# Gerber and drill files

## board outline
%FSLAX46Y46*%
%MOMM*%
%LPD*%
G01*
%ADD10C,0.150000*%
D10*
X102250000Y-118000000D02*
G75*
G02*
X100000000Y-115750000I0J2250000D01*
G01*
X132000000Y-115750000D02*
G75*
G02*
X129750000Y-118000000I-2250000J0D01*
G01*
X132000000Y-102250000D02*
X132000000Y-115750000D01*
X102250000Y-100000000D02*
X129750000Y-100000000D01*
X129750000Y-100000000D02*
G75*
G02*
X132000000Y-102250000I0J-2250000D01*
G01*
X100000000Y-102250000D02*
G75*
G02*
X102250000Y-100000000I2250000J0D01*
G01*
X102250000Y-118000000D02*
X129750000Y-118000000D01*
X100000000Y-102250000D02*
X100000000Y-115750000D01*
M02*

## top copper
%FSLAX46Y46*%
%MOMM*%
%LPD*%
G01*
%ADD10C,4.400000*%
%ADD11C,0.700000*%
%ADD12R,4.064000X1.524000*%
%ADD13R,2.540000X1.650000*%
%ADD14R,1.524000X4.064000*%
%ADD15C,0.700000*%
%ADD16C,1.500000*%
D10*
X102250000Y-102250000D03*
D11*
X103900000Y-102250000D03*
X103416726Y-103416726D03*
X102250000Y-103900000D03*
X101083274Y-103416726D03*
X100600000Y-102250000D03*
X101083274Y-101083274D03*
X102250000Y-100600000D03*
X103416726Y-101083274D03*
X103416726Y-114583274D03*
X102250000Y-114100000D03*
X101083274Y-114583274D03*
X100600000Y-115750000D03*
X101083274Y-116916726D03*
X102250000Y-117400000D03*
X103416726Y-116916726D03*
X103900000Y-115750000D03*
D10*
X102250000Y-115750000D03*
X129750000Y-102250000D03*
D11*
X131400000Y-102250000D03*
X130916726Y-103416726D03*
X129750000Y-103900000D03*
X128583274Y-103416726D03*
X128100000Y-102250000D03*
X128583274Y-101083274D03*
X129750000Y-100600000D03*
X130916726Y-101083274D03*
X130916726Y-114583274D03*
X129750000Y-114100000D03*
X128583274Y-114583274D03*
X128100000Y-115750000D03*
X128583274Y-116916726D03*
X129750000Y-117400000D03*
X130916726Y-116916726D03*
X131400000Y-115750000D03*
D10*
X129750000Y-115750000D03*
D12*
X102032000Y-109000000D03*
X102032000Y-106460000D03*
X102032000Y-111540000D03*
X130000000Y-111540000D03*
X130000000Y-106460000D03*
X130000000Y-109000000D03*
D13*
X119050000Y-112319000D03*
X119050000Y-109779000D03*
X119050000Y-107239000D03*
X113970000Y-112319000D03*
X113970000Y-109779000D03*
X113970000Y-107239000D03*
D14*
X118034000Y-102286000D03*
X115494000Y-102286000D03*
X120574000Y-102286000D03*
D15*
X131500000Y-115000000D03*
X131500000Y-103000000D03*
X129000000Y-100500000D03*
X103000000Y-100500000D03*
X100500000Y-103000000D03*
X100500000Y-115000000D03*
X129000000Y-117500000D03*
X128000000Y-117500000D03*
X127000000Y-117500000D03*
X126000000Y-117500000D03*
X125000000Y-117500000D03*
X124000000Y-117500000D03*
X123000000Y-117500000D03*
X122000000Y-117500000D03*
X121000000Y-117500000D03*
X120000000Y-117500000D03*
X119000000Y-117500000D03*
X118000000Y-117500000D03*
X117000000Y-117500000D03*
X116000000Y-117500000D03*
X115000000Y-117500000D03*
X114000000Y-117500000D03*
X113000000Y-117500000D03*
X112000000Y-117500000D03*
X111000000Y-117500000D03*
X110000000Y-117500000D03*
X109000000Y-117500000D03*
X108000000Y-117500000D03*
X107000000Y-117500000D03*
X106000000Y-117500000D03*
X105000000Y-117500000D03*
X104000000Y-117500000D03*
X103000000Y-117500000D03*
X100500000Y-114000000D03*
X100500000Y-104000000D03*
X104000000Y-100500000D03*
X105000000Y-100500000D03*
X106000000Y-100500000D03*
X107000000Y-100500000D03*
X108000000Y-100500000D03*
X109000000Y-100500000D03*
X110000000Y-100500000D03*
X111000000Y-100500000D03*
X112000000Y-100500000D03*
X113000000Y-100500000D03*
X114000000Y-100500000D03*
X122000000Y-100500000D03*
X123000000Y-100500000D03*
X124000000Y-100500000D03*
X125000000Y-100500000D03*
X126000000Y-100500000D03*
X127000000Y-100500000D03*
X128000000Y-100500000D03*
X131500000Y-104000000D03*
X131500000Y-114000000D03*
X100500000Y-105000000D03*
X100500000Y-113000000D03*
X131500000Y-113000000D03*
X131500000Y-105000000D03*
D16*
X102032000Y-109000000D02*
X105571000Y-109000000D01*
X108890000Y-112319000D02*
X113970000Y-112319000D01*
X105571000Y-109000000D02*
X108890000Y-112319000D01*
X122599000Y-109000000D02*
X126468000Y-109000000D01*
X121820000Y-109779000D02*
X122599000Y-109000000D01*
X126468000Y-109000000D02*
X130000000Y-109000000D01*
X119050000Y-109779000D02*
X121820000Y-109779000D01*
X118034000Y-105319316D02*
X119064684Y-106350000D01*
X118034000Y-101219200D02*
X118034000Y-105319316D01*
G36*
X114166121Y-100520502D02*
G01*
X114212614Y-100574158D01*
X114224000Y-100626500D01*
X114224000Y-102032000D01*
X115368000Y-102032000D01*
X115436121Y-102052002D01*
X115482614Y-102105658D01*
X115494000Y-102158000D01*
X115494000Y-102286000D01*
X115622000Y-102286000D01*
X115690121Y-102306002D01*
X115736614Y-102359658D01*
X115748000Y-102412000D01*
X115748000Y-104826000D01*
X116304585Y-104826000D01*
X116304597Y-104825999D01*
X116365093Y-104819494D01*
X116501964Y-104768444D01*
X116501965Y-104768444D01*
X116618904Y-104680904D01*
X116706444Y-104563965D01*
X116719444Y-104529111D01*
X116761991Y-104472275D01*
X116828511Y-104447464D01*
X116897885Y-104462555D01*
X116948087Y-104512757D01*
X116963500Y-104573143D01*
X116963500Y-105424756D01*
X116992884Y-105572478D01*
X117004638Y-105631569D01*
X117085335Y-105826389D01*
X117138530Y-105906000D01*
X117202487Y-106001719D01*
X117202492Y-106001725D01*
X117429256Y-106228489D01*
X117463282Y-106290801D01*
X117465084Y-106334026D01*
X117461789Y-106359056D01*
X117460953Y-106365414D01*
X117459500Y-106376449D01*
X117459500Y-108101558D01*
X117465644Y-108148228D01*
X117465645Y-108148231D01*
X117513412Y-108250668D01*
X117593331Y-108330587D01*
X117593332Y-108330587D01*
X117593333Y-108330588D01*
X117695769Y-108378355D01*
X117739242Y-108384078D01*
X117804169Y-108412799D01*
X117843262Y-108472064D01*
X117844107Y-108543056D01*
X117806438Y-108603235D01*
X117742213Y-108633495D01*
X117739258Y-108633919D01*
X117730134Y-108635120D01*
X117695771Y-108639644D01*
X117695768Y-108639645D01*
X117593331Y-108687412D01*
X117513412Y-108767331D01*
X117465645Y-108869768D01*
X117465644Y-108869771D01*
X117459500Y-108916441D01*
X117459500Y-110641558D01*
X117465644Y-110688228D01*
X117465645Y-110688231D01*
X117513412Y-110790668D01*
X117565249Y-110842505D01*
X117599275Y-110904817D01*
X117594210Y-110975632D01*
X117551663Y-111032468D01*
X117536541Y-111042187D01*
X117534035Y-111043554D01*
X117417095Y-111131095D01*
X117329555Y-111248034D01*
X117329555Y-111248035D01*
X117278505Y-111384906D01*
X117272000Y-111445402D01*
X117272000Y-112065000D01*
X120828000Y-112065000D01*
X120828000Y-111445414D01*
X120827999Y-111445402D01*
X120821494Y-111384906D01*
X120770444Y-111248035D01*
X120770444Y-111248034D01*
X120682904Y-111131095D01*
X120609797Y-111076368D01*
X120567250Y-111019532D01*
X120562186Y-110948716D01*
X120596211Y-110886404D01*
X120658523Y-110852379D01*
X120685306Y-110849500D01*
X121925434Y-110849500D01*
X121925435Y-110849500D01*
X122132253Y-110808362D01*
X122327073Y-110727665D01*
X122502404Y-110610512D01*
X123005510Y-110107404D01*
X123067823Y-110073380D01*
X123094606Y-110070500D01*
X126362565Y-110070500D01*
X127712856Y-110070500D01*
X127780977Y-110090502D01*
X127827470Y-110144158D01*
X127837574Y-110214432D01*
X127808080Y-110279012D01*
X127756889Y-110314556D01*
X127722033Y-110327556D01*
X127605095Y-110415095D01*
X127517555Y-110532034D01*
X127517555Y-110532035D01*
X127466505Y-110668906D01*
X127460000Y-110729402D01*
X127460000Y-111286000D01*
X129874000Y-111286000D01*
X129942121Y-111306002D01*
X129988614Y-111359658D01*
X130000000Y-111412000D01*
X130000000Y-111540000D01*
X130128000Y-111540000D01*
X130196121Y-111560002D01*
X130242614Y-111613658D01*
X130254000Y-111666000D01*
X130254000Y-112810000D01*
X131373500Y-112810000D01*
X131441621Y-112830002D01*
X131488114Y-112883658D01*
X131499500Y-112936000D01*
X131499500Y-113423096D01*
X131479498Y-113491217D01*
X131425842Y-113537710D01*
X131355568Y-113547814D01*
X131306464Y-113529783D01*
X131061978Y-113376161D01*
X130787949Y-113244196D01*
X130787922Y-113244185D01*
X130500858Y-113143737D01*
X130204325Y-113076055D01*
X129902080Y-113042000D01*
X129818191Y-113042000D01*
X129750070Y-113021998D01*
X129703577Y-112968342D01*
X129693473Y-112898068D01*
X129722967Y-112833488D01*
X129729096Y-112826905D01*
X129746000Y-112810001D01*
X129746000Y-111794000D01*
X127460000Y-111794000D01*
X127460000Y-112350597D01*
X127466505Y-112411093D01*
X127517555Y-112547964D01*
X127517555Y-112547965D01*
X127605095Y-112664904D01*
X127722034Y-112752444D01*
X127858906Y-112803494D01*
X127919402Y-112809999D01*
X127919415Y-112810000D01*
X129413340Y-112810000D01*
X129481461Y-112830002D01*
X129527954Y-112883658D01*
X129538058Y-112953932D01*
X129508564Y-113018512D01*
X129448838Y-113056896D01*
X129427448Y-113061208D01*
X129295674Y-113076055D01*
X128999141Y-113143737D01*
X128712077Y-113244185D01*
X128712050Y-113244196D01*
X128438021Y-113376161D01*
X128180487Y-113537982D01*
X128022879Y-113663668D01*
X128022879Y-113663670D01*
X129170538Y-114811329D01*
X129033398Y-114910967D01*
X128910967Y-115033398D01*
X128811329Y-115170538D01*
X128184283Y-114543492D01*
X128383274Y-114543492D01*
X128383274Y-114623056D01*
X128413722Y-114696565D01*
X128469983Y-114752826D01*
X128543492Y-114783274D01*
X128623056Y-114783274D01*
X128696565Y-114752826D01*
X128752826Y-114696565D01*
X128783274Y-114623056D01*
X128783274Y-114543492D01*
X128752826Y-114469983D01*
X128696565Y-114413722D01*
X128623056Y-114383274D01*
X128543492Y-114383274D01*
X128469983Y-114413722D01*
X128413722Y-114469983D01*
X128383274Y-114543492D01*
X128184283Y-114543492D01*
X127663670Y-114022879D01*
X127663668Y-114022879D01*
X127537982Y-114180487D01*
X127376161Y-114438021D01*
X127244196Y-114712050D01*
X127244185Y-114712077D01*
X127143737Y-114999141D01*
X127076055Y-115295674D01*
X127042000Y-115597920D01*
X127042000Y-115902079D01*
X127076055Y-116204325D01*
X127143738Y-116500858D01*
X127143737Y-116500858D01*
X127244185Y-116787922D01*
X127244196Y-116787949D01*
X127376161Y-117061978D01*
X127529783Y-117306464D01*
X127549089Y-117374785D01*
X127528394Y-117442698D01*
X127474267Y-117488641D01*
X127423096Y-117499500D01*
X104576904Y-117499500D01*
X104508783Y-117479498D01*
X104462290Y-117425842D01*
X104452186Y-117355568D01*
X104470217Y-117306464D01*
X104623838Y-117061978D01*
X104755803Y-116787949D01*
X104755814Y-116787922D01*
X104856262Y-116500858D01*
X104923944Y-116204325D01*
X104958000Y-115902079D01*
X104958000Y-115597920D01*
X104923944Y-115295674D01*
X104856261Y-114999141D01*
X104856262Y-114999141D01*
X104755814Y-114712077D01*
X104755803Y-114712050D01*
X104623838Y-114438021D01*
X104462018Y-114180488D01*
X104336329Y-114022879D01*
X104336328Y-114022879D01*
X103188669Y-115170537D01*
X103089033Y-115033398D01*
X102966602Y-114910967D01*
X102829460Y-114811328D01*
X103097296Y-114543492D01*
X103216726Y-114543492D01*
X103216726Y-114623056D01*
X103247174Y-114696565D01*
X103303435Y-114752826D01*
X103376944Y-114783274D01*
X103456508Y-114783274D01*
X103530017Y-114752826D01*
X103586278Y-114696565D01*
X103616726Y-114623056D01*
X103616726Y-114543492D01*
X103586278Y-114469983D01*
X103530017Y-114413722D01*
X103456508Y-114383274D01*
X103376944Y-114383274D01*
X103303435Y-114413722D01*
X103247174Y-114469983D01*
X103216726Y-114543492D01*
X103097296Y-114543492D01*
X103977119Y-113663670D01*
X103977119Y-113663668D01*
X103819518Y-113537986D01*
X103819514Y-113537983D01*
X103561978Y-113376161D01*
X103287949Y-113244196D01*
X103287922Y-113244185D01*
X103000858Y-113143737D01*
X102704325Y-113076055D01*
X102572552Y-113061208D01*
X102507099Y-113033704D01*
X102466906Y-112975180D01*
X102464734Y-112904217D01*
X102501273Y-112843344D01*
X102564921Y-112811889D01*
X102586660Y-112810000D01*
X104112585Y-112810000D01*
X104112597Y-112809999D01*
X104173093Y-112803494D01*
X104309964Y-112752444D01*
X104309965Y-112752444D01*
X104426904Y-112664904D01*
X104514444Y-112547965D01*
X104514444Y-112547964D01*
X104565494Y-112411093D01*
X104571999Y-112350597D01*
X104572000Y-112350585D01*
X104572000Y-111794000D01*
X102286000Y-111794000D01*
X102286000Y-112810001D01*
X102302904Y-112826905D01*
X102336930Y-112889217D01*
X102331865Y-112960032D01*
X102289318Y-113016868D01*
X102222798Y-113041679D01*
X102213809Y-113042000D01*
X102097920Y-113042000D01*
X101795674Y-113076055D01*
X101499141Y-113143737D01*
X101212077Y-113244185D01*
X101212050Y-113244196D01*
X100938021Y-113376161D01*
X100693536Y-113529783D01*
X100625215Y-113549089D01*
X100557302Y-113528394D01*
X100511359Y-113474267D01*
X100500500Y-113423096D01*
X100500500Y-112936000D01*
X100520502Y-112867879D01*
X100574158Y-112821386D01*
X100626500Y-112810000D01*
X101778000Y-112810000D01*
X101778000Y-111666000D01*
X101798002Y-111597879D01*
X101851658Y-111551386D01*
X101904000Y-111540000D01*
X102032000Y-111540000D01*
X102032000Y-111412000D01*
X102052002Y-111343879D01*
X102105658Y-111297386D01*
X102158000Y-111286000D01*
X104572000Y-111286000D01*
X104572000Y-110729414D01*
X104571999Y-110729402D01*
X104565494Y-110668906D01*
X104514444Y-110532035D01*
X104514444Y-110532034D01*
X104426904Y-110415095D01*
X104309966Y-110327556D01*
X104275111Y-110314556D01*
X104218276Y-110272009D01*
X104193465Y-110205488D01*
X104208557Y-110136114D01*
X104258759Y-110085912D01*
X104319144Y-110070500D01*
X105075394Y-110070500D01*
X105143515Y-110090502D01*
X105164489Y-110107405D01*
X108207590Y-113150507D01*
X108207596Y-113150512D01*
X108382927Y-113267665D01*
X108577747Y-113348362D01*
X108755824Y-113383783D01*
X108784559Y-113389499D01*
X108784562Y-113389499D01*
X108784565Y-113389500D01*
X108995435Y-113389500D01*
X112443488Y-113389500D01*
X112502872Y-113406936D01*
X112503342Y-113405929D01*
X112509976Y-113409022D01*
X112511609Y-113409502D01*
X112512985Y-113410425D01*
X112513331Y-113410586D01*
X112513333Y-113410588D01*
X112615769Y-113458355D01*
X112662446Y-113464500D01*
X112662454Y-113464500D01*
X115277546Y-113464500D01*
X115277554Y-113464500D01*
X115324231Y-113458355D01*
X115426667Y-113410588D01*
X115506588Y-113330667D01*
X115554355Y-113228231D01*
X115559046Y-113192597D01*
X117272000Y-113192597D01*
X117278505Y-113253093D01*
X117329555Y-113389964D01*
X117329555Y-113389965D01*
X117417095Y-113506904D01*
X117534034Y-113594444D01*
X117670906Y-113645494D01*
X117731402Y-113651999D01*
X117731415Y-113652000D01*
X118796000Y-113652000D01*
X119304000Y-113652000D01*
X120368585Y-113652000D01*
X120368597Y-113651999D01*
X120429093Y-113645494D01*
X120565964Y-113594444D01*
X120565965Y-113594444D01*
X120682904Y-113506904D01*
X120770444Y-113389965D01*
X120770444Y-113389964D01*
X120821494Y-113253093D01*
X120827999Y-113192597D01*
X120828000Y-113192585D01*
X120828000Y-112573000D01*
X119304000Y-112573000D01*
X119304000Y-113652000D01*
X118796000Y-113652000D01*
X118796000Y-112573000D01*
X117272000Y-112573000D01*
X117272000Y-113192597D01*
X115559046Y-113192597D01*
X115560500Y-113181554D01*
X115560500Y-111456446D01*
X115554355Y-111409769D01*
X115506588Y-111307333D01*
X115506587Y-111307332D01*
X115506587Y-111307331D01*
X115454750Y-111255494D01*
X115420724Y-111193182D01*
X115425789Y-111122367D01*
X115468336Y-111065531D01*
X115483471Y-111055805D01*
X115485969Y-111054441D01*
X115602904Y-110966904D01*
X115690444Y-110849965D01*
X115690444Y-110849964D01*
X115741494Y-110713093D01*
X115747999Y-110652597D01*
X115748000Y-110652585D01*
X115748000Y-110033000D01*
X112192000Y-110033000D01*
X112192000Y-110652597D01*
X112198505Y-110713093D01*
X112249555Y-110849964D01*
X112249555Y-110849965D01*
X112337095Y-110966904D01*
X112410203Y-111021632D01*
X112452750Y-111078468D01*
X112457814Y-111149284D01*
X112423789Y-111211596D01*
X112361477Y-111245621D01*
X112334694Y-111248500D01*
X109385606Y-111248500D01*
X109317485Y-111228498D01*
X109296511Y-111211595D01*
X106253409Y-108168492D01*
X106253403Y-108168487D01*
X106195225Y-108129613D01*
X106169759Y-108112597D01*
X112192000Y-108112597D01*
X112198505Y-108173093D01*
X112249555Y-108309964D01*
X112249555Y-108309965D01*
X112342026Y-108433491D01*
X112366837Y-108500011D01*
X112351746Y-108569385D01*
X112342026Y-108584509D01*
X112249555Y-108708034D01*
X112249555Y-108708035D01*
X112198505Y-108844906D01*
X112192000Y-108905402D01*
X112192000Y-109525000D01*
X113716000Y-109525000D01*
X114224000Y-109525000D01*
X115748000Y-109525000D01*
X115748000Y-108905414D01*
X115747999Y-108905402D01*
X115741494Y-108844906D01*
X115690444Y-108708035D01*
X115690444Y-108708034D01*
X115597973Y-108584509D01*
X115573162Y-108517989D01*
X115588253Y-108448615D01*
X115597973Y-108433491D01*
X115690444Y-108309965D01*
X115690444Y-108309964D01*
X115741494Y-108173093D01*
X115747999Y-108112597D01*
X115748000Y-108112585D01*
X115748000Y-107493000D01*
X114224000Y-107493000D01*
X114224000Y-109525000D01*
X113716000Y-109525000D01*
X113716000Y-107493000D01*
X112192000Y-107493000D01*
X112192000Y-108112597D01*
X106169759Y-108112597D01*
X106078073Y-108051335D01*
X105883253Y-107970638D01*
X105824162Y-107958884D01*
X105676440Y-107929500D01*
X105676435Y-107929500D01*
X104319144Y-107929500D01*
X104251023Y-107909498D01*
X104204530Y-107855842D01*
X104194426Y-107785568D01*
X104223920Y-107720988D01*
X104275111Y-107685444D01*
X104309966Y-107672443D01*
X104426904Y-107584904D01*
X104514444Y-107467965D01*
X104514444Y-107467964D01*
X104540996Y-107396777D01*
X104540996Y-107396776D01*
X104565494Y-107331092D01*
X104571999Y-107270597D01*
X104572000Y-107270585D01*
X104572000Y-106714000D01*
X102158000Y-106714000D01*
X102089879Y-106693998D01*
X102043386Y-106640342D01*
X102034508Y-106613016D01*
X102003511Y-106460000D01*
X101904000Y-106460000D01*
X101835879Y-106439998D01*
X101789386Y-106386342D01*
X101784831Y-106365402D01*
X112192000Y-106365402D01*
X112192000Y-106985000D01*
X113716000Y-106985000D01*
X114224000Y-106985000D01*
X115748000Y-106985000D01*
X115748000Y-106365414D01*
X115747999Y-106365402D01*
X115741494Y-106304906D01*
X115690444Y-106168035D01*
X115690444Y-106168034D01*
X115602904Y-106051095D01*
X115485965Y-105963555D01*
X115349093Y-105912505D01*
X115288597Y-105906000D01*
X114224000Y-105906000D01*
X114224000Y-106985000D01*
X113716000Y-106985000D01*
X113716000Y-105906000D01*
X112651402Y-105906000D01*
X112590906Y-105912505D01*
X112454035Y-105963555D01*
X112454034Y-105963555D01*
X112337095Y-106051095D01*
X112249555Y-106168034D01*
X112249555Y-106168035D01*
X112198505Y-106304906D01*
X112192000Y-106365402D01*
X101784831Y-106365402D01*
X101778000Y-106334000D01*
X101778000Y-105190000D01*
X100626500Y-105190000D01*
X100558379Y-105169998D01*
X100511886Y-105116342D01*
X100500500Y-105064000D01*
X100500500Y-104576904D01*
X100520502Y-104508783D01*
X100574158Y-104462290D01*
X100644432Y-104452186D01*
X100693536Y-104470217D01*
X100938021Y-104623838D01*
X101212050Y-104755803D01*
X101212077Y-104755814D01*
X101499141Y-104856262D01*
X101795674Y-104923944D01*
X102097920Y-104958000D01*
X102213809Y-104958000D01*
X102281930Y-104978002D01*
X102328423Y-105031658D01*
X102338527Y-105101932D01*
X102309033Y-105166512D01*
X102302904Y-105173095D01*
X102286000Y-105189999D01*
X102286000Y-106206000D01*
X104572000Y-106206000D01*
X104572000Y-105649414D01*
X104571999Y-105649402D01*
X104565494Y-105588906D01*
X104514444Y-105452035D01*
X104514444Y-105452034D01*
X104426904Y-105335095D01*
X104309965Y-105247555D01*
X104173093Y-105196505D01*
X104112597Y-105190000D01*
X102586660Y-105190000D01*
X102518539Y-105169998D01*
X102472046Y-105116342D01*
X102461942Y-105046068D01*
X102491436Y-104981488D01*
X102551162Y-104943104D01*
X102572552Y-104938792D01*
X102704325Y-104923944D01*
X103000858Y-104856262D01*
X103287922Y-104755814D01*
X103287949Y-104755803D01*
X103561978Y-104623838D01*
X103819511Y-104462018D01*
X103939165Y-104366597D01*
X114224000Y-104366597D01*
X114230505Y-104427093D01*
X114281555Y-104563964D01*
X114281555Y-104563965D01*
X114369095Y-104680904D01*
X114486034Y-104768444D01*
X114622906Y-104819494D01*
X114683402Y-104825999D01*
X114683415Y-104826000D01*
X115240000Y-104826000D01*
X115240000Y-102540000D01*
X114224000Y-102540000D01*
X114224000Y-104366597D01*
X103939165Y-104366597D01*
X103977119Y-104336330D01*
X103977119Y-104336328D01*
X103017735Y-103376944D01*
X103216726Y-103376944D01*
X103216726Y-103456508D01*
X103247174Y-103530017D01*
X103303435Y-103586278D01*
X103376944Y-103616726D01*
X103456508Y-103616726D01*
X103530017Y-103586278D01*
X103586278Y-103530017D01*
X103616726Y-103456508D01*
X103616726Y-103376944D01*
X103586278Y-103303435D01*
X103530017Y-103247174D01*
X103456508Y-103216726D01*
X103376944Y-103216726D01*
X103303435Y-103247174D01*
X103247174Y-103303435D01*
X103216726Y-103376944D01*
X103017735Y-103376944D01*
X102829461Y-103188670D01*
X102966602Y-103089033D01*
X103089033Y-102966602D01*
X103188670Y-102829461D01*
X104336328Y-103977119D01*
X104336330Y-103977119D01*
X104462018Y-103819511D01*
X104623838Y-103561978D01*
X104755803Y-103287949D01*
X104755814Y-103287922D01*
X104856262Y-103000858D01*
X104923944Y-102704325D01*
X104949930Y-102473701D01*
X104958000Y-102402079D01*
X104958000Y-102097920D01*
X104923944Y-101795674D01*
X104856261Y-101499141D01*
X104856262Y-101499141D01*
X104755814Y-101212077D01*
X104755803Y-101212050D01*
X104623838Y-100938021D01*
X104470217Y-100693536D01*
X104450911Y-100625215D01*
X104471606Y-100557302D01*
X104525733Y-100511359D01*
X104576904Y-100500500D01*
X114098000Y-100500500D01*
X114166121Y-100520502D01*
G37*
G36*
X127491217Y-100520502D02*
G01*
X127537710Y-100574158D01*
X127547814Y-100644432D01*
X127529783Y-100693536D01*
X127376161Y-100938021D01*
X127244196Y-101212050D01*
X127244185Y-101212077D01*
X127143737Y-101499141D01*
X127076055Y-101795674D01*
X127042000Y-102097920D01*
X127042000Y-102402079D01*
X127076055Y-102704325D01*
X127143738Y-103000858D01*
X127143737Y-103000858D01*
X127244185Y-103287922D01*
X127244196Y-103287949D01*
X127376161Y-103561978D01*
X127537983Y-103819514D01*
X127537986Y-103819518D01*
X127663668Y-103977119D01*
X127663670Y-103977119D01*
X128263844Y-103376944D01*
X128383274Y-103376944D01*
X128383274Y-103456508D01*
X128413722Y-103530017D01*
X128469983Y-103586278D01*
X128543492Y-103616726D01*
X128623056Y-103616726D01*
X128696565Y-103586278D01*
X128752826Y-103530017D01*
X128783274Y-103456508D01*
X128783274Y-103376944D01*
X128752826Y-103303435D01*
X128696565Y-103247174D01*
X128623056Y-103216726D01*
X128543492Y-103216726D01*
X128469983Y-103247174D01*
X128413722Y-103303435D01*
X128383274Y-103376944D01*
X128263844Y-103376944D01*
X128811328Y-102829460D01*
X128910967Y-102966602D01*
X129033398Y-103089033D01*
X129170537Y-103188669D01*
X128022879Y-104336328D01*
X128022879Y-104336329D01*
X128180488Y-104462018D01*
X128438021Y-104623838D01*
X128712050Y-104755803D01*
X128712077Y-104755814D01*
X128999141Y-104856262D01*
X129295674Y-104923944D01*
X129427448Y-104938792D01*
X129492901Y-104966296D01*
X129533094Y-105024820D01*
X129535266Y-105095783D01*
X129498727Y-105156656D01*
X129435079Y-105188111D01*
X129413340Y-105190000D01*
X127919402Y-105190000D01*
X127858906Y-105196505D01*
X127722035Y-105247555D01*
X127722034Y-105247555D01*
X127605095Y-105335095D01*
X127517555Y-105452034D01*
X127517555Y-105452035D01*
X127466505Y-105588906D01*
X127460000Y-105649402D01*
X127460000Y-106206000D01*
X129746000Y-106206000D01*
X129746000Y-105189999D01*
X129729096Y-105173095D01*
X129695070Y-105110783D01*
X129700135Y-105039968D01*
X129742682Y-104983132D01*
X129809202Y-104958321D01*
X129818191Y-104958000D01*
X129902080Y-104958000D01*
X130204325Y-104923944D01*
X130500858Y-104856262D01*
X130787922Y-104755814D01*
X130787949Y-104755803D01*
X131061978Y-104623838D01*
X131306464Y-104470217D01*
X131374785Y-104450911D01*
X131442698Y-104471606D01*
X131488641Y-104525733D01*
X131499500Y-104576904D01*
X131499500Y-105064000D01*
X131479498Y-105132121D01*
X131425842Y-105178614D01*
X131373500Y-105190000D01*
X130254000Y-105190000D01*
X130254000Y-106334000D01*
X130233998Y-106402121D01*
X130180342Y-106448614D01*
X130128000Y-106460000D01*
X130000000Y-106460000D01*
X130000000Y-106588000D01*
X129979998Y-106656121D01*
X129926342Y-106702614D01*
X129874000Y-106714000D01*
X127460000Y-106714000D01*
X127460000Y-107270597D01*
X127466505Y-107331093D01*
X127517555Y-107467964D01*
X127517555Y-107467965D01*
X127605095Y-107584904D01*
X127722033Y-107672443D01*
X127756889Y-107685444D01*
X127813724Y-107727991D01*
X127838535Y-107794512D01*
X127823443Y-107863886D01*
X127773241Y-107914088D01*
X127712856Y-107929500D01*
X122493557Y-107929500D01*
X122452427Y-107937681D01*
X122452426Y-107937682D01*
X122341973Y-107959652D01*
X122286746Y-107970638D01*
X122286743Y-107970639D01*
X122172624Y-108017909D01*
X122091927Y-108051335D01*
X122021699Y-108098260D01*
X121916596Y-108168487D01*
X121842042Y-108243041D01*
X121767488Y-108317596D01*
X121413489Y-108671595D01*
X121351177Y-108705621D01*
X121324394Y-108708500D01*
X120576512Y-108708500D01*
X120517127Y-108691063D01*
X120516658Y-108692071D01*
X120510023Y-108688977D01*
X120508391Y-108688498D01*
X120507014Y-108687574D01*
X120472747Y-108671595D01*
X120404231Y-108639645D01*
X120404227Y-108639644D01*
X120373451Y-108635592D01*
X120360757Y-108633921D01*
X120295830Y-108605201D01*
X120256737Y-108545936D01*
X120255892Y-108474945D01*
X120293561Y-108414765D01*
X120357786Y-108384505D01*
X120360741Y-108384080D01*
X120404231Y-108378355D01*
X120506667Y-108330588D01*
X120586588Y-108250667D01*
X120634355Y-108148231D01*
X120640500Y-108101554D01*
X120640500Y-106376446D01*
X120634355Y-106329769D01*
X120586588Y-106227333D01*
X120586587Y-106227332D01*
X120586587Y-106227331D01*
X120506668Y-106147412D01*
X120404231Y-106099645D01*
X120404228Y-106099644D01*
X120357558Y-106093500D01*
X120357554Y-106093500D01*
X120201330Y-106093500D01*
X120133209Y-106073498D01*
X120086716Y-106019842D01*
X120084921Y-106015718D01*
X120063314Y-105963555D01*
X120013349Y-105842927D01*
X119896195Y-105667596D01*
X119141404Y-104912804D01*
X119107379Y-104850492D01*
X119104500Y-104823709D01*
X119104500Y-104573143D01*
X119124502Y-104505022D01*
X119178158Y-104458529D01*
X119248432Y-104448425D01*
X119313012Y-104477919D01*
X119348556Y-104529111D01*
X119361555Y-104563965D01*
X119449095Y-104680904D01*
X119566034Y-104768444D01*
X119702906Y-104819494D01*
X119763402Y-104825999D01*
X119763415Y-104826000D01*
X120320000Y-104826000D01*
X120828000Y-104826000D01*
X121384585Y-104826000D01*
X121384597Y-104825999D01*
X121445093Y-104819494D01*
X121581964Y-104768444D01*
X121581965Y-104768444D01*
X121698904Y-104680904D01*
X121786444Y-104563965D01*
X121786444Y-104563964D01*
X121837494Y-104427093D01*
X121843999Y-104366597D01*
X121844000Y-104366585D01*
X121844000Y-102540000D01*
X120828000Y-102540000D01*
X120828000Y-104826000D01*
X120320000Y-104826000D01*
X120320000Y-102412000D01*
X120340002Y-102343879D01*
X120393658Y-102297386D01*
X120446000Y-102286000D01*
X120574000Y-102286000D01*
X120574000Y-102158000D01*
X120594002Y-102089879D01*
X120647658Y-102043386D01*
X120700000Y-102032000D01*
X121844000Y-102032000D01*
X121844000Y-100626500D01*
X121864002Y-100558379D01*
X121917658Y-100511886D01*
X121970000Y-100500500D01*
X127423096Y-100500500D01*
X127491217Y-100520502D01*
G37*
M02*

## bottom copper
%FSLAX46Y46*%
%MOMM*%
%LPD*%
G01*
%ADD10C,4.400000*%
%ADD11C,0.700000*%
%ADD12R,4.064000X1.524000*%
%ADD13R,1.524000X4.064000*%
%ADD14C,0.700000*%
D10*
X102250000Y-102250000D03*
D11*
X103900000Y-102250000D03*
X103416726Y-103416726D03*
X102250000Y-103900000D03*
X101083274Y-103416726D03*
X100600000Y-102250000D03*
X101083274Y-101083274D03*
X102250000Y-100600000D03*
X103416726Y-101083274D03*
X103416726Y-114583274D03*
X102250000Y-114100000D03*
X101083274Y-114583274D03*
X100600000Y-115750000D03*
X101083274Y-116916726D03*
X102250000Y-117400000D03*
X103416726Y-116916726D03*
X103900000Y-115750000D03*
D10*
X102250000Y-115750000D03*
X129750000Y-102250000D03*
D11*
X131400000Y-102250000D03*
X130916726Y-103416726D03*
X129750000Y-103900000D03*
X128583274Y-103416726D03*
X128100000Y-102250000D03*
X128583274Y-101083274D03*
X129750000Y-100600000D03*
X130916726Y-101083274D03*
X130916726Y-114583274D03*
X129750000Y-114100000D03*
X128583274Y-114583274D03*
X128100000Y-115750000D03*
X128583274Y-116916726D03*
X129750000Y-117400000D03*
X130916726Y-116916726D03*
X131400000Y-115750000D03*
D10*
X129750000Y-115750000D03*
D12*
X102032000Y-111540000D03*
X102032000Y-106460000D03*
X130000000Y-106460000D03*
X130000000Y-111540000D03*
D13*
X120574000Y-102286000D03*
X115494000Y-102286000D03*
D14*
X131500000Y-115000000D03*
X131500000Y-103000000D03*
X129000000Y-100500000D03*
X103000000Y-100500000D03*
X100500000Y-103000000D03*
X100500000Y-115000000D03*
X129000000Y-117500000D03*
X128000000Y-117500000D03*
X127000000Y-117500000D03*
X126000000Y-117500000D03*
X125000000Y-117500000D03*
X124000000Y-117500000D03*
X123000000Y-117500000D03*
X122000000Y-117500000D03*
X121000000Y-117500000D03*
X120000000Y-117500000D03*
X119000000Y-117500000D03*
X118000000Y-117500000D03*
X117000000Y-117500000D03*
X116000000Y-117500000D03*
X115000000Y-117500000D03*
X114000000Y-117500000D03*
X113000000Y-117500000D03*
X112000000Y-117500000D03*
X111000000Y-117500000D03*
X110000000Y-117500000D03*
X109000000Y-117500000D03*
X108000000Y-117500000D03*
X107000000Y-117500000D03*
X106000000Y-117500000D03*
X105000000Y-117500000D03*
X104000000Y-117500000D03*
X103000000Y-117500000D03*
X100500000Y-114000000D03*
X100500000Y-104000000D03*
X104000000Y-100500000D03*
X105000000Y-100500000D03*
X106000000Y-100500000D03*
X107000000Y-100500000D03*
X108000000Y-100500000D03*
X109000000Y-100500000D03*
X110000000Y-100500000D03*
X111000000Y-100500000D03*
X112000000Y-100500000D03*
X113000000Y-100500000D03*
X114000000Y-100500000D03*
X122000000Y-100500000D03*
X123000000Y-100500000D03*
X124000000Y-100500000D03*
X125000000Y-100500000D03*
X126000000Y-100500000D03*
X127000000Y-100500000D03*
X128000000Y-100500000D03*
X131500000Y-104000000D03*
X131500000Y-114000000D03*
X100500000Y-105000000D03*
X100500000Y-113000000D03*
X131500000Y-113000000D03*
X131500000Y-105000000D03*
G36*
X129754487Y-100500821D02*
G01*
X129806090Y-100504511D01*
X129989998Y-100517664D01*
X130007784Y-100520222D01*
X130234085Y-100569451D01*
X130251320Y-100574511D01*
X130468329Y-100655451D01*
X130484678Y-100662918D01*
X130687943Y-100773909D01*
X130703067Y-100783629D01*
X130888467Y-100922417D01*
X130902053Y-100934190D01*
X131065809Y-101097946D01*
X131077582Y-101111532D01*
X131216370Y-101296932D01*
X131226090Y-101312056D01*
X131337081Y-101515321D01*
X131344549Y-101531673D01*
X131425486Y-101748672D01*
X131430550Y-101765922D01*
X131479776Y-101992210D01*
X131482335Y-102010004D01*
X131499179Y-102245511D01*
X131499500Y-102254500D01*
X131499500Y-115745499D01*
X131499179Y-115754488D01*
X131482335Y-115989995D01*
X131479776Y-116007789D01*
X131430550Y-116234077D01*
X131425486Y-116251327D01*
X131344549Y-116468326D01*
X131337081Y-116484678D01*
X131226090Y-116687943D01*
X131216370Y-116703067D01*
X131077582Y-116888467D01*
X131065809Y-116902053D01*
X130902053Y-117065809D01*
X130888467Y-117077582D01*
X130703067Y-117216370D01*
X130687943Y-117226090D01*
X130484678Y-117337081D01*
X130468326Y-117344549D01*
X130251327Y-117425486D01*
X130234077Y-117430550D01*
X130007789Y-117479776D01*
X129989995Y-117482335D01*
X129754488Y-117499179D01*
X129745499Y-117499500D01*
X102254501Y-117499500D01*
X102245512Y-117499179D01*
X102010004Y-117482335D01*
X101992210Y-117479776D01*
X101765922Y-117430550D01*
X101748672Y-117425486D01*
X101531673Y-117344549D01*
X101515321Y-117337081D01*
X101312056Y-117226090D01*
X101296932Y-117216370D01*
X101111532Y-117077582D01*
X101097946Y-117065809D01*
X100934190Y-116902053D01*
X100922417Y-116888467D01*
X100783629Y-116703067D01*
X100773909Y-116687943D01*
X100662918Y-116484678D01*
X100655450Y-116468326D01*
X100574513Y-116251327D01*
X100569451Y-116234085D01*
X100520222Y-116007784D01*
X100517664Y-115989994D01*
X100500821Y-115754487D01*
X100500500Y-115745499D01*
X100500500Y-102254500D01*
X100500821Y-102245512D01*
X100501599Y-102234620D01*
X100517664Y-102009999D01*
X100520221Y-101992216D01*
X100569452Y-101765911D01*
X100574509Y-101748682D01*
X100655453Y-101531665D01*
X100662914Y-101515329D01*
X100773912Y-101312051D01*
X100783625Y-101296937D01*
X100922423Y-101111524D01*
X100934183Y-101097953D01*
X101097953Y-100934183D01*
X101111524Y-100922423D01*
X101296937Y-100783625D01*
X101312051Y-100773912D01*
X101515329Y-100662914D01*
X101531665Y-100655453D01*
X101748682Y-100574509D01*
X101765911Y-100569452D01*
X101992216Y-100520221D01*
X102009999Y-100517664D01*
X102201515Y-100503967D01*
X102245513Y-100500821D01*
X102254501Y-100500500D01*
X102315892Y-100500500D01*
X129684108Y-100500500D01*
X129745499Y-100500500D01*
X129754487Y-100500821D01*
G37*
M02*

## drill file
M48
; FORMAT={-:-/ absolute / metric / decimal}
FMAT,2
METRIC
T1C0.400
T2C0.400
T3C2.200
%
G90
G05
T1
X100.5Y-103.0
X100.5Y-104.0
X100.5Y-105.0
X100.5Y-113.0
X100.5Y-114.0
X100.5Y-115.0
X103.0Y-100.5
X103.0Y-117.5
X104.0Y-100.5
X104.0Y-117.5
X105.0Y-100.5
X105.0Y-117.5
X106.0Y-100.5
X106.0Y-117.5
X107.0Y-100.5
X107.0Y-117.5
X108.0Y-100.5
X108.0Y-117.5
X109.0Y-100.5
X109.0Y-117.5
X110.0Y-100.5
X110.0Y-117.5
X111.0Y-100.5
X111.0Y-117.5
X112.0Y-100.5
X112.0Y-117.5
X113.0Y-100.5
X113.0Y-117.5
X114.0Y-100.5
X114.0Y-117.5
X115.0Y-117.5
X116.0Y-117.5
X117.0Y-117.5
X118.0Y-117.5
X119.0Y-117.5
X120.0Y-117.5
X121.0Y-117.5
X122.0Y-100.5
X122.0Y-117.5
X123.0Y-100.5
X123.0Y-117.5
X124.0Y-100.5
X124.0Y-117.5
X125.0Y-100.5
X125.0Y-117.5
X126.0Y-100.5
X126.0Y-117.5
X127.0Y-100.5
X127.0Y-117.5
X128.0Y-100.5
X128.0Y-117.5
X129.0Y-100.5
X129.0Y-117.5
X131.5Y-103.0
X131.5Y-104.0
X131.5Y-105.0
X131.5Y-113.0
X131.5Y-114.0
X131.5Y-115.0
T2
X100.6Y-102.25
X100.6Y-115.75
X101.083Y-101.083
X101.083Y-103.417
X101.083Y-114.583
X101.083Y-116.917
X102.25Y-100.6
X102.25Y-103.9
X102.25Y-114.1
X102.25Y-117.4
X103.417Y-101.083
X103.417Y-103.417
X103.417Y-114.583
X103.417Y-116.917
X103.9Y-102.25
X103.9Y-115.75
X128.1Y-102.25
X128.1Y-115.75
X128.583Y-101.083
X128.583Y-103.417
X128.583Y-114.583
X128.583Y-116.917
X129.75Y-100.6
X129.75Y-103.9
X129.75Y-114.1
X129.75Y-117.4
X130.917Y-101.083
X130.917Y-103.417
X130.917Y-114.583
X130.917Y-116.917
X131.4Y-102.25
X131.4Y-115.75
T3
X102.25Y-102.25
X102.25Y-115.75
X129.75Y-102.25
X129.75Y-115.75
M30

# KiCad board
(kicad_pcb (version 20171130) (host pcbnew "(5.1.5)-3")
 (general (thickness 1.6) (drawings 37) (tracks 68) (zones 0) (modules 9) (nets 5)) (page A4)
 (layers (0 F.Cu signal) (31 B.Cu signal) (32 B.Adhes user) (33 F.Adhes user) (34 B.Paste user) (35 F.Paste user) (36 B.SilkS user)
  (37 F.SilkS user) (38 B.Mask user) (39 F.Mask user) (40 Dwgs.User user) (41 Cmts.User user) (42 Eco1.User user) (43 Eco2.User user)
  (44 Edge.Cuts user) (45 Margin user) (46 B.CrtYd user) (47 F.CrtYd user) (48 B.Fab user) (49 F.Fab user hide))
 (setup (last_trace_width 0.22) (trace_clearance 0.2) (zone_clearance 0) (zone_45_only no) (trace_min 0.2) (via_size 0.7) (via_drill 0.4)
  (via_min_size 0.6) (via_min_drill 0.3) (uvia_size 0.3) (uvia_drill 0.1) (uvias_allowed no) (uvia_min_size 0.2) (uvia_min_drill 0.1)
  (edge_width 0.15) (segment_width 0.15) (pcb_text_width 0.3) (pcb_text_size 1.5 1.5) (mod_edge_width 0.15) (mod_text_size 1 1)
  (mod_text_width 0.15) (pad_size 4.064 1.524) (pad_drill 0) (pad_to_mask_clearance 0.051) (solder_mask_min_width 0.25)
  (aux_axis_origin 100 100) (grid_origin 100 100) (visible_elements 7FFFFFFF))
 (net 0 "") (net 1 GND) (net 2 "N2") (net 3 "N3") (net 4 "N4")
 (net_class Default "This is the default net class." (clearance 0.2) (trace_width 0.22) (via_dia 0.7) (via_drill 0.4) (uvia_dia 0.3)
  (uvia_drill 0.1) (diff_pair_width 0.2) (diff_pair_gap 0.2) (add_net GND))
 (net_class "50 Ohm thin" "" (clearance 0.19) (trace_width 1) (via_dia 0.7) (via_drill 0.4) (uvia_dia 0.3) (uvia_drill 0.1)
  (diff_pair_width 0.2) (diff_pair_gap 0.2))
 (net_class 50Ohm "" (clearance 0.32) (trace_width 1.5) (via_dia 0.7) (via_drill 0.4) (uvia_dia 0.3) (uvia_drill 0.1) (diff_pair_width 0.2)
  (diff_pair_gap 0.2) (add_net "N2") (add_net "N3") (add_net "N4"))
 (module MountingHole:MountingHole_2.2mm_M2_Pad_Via (layer F.Cu) (at 102.25 102.25)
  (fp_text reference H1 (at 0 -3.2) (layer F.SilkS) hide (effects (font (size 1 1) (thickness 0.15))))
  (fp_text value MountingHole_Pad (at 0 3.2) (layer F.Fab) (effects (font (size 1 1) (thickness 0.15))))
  (pad 1 thru_hole circle (at 0 0) (size 4.4 4.4) (drill 2.2) (layers *.Cu *.Mask) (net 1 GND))
  (pad 1 thru_hole circle (at 1.65 0) (size 0.7 0.7) (drill 0.4) (layers *.Cu *.Mask) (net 1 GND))
  (pad 1 thru_hole circle (at 1.166726 1.166726) (size 0.7 0.7) (drill 0.4) (layers *.Cu *.Mask) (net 1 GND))
  (pad 1 thru_hole circle (at 0 1.65) (size 0.7 0.7) (drill 0.4) (layers *.Cu *.Mask) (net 1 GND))
  (pad 1 thru_hole circle (at -1.166726 1.166726) (size 0.7 0.7) (drill 0.4) (layers *.Cu *.Mask) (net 1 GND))
  (pad 1 thru_hole circle (at -1.65 0) (size 0.7 0.7) (drill 0.4) (layers *.Cu *.Mask) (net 1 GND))
  (pad 1 thru_hole circle (at -1.166726 -1.166726) (size 0.7 0.7) (drill 0.4) (layers *.Cu *.Mask) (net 1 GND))
  (pad 1 thru_hole circle (at 0 -1.65) (size 0.7 0.7) (drill 0.4) (layers *.Cu *.Mask) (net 1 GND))
  (pad 1 thru_hole circle (at 1.166726 -1.166726) (size 0.7 0.7) (drill 0.4) (layers *.Cu *.Mask) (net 1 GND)))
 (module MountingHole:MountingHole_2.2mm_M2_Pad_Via (layer F.Cu) (at 102.25 115.75)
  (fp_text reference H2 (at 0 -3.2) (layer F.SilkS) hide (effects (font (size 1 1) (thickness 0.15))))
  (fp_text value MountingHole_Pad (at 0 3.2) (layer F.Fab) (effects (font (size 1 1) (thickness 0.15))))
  (pad 1 thru_hole circle (at 1.166726 -1.166726) (size 0.7 0.7) (drill 0.4) (layers *.Cu *.Mask) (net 1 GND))
  (pad 1 thru_hole circle (at 0 -1.65) (size 0.7 0.7) (drill 0.4) (layers *.Cu *.Mask) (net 1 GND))
  (pad 1 thru_hole circle (at -1.166726 -1.166726) (size 0.7 0.7) (drill 0.4) (layers *.Cu *.Mask) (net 1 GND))
  (pad 1 thru_hole circle (at -1.65 0) (size 0.7 0.7) (drill 0.4) (layers *.Cu *.Mask) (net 1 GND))
  (pad 1 thru_hole circle (at -1.166726 1.166726) (size 0.7 0.7) (drill 0.4) (layers *.Cu *.Mask) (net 1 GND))
  (pad 1 thru_hole circle (at 0 1.65) (size 0.7 0.7) (drill 0.4) (layers *.Cu *.Mask) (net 1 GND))
  (pad 1 thru_hole circle (at 1.166726 1.166726) (size 0.7 0.7) (drill 0.4) (layers *.Cu *.Mask) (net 1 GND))
  (pad 1 thru_hole circle (at 1.65 0) (size 0.7 0.7) (drill 0.4) (layers *.Cu *.Mask) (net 1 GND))
  (pad 1 thru_hole circle (at 0 0) (size 4.4 4.4) (drill 2.2) (layers *.Cu *.Mask) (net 1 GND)))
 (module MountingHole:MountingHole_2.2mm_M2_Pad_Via (layer F.Cu) (at 129.75 102.25)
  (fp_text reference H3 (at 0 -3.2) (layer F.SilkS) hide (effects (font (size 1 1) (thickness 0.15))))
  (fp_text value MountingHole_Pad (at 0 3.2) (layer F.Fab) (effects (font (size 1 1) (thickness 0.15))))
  (pad 1 thru_hole circle (at 0 0) (size 4.4 4.4) (drill 2.2) (layers *.Cu *.Mask) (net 1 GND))
  (pad 1 thru_hole circle (at 1.65 0) (size 0.7 0.7) (drill 0.4) (layers *.Cu *.Mask) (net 1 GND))
  (pad 1 thru_hole circle (at 1.166726 1.166726) (size 0.7 0.7) (drill 0.4) (layers *.Cu *.Mask) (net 1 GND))
  (pad 1 thru_hole circle (at 0 1.65) (size 0.7 0.7) (drill 0.4) (layers *.Cu *.Mask) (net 1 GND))
  (pad 1 thru_hole circle (at -1.166726 1.166726) (size 0.7 0.7) (drill 0.4) (layers *.Cu *.Mask) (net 1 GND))
  (pad 1 thru_hole circle (at -1.65 0) (size 0.7 0.7) (drill 0.4) (layers *.Cu *.Mask) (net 1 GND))
  (pad 1 thru_hole circle (at -1.166726 -1.166726) (size 0.7 0.7) (drill 0.4) (layers *.Cu *.Mask) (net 1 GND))
  (pad 1 thru_hole circle (at 0 -1.65) (size 0.7 0.7) (drill 0.4) (layers *.Cu *.Mask) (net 1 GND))
  (pad 1 thru_hole circle (at 1.166726 -1.166726) (size 0.7 0.7) (drill 0.4) (layers *.Cu *.Mask) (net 1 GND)))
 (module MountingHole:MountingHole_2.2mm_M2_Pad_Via (layer F.Cu) (at 129.75 115.75)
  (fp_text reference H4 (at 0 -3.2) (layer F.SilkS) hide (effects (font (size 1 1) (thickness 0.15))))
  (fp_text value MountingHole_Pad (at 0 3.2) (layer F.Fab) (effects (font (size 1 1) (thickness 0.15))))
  (pad 1 thru_hole circle (at 1.166726 -1.166726) (size 0.7 0.7) (drill 0.4) (layers *.Cu *.Mask) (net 1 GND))
  (pad 1 thru_hole circle (at 0 -1.65) (size 0.7 0.7) (drill 0.4) (layers *.Cu *.Mask) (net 1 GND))
  (pad 1 thru_hole circle (at -1.166726 -1.166726) (size 0.7 0.7) (drill 0.4) (layers *.Cu *.Mask) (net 1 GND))
  (pad 1 thru_hole circle (at -1.65 0) (size 0.7 0.7) (drill 0.4) (layers *.Cu *.Mask) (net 1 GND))
  (pad 1 thru_hole circle (at -1.166726 1.166726) (size 0.7 0.7) (drill 0.4) (layers *.Cu *.Mask) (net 1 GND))
  (pad 1 thru_hole circle (at 0 1.65) (size 0.7 0.7) (drill 0.4) (layers *.Cu *.Mask) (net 1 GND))
  (pad 1 thru_hole circle (at 1.166726 1.166726) (size 0.7 0.7) (drill 0.4) (layers *.Cu *.Mask) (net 1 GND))
  (pad 1 thru_hole circle (at 1.65 0) (size 0.7 0.7) (drill 0.4) (layers *.Cu *.Mask) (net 1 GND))
  (pad 1 thru_hole circle (at 0 0) (size 4.4 4.4) (drill 2.2) (layers *.Cu *.Mask) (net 1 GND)))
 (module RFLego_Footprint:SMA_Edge (layer F.Cu) (at 100 109)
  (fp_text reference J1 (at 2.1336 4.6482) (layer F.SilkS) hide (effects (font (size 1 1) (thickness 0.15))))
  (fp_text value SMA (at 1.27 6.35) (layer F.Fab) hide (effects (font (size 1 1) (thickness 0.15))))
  (pad 1 smd rect (at 2.032 0) (size 4.064 1.524) (layers F.Cu F.Mask) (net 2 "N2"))
  (pad 2 smd rect (at 2.032 -2.54) (size 4.064 1.524) (layers F.Cu F.Mask) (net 1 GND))
  (pad 2 smd rect (at 2.032 2.54) (size 4.064 1.524) (layers B.Cu B.Mask) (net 1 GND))
  (pad 2 smd rect (at 2.032 -2.54) (size 4.064 1.524) (layers B.Cu B.Mask) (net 1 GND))
  (pad 2 smd rect (at 2.032 2.54) (size 4.064 1.524) (layers F.Cu F.Mask) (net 1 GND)))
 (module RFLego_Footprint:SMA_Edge (layer F.Cu) (at 127.968 109)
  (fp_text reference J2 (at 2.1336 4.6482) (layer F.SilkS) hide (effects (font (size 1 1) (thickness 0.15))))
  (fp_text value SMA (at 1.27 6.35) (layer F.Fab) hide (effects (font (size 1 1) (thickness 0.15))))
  (pad 2 smd rect (at 2.032 2.54) (size 4.064 1.524) (layers F.Cu F.Mask) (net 1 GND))
  (pad 2 smd rect (at 2.032 -2.54) (size 4.064 1.524) (layers B.Cu B.Mask) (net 1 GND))
  (pad 2 smd rect (at 2.032 2.54) (size 4.064 1.524) (layers B.Cu B.Mask) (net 1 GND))
  (pad 2 smd rect (at 2.032 -2.54) (size 4.064 1.524) (layers F.Cu F.Mask) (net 1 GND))
  (pad 1 smd rect (at 2.032 0) (size 4.064 1.524) (layers F.Cu F.Mask) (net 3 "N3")))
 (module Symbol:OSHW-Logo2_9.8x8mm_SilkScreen (layer B.Cu) (at 109.5 113.25 180)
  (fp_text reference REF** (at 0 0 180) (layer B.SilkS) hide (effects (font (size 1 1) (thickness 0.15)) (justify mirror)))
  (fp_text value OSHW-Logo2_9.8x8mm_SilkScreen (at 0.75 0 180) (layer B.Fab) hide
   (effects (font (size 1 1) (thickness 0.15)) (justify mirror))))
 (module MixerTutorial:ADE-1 (layer F.Cu) (at 119.05 112.319 90)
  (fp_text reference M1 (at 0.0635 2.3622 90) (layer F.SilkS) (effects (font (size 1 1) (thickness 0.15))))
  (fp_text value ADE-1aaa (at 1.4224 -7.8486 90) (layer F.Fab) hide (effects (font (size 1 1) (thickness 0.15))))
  (pad 4 smd rect (at 0 0 90) (size 1.65 2.54) (layers F.Cu F.Paste F.Mask) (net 1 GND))
  (pad 3 smd rect (at 2.54 0 90) (size 1.65 2.54) (layers F.Cu F.Paste F.Mask) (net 3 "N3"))
  (pad 2 smd rect (at 5.08 0 90) (size 1.65 2.54) (layers F.Cu F.Paste F.Mask) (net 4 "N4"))
  (pad 1 smd rect (at 0 -5.08 90) (size 1.65 2.54) (layers F.Cu F.Paste F.Mask) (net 2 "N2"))
  (pad 4 smd rect (at 2.54 -5.08 90) (size 1.65 2.54) (layers F.Cu F.Paste F.Mask) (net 1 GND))
  (pad 4 smd rect (at 5.08 -5.08 90) (size 1.65 2.54) (layers F.Cu F.Paste F.Mask) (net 1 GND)))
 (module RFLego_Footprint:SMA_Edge (layer F.Cu) (at 118.034 104.318 90)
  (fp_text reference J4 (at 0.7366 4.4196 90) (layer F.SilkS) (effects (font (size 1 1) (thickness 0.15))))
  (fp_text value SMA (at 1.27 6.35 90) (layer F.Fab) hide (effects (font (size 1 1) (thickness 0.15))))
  (pad 1 smd rect (at 2.032 0 90) (size 4.064 1.524) (layers F.Cu F.Mask) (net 4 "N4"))
  (pad 2 smd rect (at 2.032 -2.54 90) (size 4.064 1.524) (layers F.Cu F.Mask) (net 1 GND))
  (pad 2 smd rect (at 2.032 2.54 90) (size 4.064 1.524) (layers B.Cu B.Mask) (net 1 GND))
  (pad 2 smd rect (at 2.032 -2.54 90) (size 4.064 1.524) (layers B.Cu B.Mask) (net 1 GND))
  (pad 2 smd rect (at 2.032 2.54 90) (size 4.064 1.524) (layers F.Cu F.Mask) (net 1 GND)))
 (gr_arc (start 102.25 115.75) (end 100 115.75) (angle -90) (layer Edge.Cuts) (width 0.15))
 (gr_arc (start 129.75 115.75) (end 129.75 118) (angle -90) (layer Edge.Cuts) (width 0.15))
 (gr_line (start 132 102.25) (end 132 115.75) (layer Edge.Cuts) (width 0.15))
 (gr_line (start 102.25 100) (end 129.75 100) (layer Edge.Cuts) (width 0.15))
 (gr_arc (start 129.75 102.25) (end 132 102.25) (angle -90) (layer Edge.Cuts) (width 0.15))
 (gr_arc (start 102.25 102.25) (end 102.25 100) (angle -90) (layer Edge.Cuts) (width 0.15))
 (gr_line (start 102.25 118) (end 129.75 118) (layer Edge.Cuts) (width 0.15))
 (gr_line (start 100 102.25) (end 100 115.75) (layer Edge.Cuts) (width 0.15))
 (via (at 131.5 115) (size 0.7) (drill 0.4) (layers F.Cu B.Cu) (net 1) (status 30))
 (via (at 131.5 103) (size 0.7) (drill 0.4) (layers F.Cu B.Cu) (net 1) (status 30))
 (via (at 129 100.5) (size 0.7) (drill 0.4) (layers F.Cu B.Cu) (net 1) (status 30))
 (via (at 103 100.5) (size 0.7) (drill 0.4) (layers F.Cu B.Cu) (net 1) (status 30))
 (via (at 100.5 103) (size 0.7) (drill 0.4) (layers F.Cu B.Cu) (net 1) (status 30))
 (via (at 100.5 115) (size 0.7) (drill 0.4) (layers F.Cu B.Cu) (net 1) (status 30))
 (via (at 129 117.5) (size 0.7) (drill 0.4) (layers F.Cu B.Cu) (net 1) (status 30))
 (via (at 128 117.5) (size 0.7) (drill 0.4) (layers F.Cu B.Cu) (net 1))
 (via (at 127 117.5) (size 0.7) (drill 0.4) (layers F.Cu B.Cu) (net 1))
 (via (at 126 117.5) (size 0.7) (drill 0.4) (layers F.Cu B.Cu) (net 1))
 (via (at 125 117.5) (size 0.7) (drill 0.4) (layers F.Cu B.Cu) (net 1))
 (via (at 124 117.5) (size 0.7) (drill 0.4) (layers F.Cu B.Cu) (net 1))
 (via (at 123 117.5) (size 0.7) (drill 0.4) (layers F.Cu B.Cu) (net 1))
 (via (at 122 117.5) (size 0.7) (drill 0.4) (layers F.Cu B.Cu) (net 1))
 (via (at 121 117.5) (size 0.7) (drill 0.4) (layers F.Cu B.Cu) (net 1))
 (via (at 120 117.5) (size 0.7) (drill 0.4) (layers F.Cu B.Cu) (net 1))
 (via (at 119 117.5) (size 0.7) (drill 0.4) (layers F.Cu B.Cu) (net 1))
 (via (at 118 117.5) (size 0.7) (drill 0.4) (layers F.Cu B.Cu) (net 1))
 (via (at 117 117.5) (size 0.7) (drill 0.4) (layers F.Cu B.Cu) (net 1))
 (via (at 116 117.5) (size 0.7) (drill 0.4) (layers F.Cu B.Cu) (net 1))
 (via (at 115 117.5) (size 0.7) (drill 0.4) (layers F.Cu B.Cu) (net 1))
 (via (at 114 117.5) (size 0.7) (drill 0.4) (layers F.Cu B.Cu) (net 1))
 (via (at 113 117.5) (size 0.7) (drill 0.4) (layers F.Cu B.Cu) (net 1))
 (via (at 112 117.5) (size 0.7) (drill 0.4) (layers F.Cu B.Cu) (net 1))
 (via (at 111 117.5) (size 0.7) (drill 0.4) (layers F.Cu B.Cu) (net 1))
 (via (at 110 117.5) (size 0.7) (drill 0.4) (layers F.Cu B.Cu) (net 1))
 (via (at 109 117.5) (size 0.7) (drill 0.4) (layers F.Cu B.Cu) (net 1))
 (via (at 108 117.5) (size 0.7) (drill 0.4) (layers F.Cu B.Cu) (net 1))
 (via (at 107 117.5) (size 0.7) (drill 0.4) (layers F.Cu B.Cu) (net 1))
 (via (at 106 117.5) (size 0.7) (drill 0.4) (layers F.Cu B.Cu) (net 1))
 (via (at 105 117.5) (size 0.7) (drill 0.4) (layers F.Cu B.Cu) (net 1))
 (via (at 104 117.5) (size 0.7) (drill 0.4) (layers F.Cu B.Cu) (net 1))
 (via (at 103 117.5) (size 0.7) (drill 0.4) (layers F.Cu B.Cu) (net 1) (status 30))
 (via (at 100.5 114) (size 0.7) (drill 0.4) (layers F.Cu B.Cu) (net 1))
 (via (at 100.5 104) (size 0.7) (drill 0.4) (layers F.Cu B.Cu) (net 1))
 (via (at 104 100.5) (size 0.7) (drill 0.4) (layers F.Cu B.Cu) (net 1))
 (via (at 105 100.5) (size 0.7) (drill 0.4) (layers F.Cu B.Cu) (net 1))
 (via (at 106 100.5) (size 0.7) (drill 0.4) (layers F.Cu B.Cu) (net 1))
 (via (at 107 100.5) (size 0.7) (drill 0.4) (layers F.Cu B.Cu) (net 1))
 (via (at 108 100.5) (size 0.7) (drill 0.4) (layers F.Cu B.Cu) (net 1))
 (via (at 109 100.5) (size 0.7) (drill 0.4) (layers F.Cu B.Cu) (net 1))
 (via (at 110 100.5) (size 0.7) (drill 0.4) (layers F.Cu B.Cu) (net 1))
 (via (at 111 100.5) (size 0.7) (drill 0.4) (layers F.Cu B.Cu) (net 1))
 (via (at 112 100.5) (size 0.7) (drill 0.4) (layers F.Cu B.Cu) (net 1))
 (via (at 113 100.5) (size 0.7) (drill 0.4) (layers F.Cu B.Cu) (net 1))
 (via (at 114 100.5) (size 0.7) (drill 0.4) (layers F.Cu B.Cu) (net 1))
 (via (at 122 100.5) (size 0.7) (drill 0.4) (layers F.Cu B.Cu) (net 1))
 (via (at 123 100.5) (size 0.7) (drill 0.4) (layers F.Cu B.Cu) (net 1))
 (via (at 124 100.5) (size 0.7) (drill 0.4) (layers F.Cu B.Cu) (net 1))
 (via (at 125 100.5) (size 0.7) (drill 0.4) (layers F.Cu B.Cu) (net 1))
 (via (at 126 100.5) (size 0.7) (drill 0.4) (layers F.Cu B.Cu) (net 1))
 (via (at 127 100.5) (size 0.7) (drill 0.4) (layers F.Cu B.Cu) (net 1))
 (via (at 128 100.5) (size 0.7) (drill 0.4) (layers F.Cu B.Cu) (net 1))
 (via (at 131.5 104) (size 0.7) (drill 0.4) (layers F.Cu B.Cu) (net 1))
 (via (at 131.5 114) (size 0.7) (drill 0.4) (layers F.Cu B.Cu) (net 1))
 (via (at 100.5 105) (size 0.7) (drill 0.4) (layers F.Cu B.Cu) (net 1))
 (via (at 100.5 113) (size 0.7) (drill 0.4) (layers F.Cu B.Cu) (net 1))
 (via (at 131.5 113) (size 0.7) (drill 0.4) (layers F.Cu B.Cu) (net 1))
 (via (at 131.5 105) (size 0.7) (drill 0.4) (layers F.Cu B.Cu) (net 1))
 (segment (start 102.032 109) (end 105.571 109) (width 1.5) (layer F.Cu) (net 2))
 (segment (start 108.89 112.319) (end 113.97 112.319) (width 1.5) (layer F.Cu) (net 2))
 (segment (start 105.571 109) (end 108.89 112.319) (width 1.5) (layer F.Cu) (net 2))
 (segment (start 122.599 109) (end 126.468 109) (width 1.5) (layer F.Cu) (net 3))
 (segment (start 121.82 109.779) (end 122.599 109) (width 1.5) (layer F.Cu) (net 3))
 (segment (start 126.468 109) (end 130 109) (width 1.5) (layer F.Cu) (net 3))
 (segment (start 119.05 109.779) (end 121.82 109.779) (width 1.5) (layer F.Cu) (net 3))
 (segment (start 118.034 105.319316) (end 119.064684 106.35) (width 1.5) (layer F.Cu) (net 4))
 (segment (start 118.034 101.2192) (end 118.034 105.319316) (width 1.5) (layer F.Cu) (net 4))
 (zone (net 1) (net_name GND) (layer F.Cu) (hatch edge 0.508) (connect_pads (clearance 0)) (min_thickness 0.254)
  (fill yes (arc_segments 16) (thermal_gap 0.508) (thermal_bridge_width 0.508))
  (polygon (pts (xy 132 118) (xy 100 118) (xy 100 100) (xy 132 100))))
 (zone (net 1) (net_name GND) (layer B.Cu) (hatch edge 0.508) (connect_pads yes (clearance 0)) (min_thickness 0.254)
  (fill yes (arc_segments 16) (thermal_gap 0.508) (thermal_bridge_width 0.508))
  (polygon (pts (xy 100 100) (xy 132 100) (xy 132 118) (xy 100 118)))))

